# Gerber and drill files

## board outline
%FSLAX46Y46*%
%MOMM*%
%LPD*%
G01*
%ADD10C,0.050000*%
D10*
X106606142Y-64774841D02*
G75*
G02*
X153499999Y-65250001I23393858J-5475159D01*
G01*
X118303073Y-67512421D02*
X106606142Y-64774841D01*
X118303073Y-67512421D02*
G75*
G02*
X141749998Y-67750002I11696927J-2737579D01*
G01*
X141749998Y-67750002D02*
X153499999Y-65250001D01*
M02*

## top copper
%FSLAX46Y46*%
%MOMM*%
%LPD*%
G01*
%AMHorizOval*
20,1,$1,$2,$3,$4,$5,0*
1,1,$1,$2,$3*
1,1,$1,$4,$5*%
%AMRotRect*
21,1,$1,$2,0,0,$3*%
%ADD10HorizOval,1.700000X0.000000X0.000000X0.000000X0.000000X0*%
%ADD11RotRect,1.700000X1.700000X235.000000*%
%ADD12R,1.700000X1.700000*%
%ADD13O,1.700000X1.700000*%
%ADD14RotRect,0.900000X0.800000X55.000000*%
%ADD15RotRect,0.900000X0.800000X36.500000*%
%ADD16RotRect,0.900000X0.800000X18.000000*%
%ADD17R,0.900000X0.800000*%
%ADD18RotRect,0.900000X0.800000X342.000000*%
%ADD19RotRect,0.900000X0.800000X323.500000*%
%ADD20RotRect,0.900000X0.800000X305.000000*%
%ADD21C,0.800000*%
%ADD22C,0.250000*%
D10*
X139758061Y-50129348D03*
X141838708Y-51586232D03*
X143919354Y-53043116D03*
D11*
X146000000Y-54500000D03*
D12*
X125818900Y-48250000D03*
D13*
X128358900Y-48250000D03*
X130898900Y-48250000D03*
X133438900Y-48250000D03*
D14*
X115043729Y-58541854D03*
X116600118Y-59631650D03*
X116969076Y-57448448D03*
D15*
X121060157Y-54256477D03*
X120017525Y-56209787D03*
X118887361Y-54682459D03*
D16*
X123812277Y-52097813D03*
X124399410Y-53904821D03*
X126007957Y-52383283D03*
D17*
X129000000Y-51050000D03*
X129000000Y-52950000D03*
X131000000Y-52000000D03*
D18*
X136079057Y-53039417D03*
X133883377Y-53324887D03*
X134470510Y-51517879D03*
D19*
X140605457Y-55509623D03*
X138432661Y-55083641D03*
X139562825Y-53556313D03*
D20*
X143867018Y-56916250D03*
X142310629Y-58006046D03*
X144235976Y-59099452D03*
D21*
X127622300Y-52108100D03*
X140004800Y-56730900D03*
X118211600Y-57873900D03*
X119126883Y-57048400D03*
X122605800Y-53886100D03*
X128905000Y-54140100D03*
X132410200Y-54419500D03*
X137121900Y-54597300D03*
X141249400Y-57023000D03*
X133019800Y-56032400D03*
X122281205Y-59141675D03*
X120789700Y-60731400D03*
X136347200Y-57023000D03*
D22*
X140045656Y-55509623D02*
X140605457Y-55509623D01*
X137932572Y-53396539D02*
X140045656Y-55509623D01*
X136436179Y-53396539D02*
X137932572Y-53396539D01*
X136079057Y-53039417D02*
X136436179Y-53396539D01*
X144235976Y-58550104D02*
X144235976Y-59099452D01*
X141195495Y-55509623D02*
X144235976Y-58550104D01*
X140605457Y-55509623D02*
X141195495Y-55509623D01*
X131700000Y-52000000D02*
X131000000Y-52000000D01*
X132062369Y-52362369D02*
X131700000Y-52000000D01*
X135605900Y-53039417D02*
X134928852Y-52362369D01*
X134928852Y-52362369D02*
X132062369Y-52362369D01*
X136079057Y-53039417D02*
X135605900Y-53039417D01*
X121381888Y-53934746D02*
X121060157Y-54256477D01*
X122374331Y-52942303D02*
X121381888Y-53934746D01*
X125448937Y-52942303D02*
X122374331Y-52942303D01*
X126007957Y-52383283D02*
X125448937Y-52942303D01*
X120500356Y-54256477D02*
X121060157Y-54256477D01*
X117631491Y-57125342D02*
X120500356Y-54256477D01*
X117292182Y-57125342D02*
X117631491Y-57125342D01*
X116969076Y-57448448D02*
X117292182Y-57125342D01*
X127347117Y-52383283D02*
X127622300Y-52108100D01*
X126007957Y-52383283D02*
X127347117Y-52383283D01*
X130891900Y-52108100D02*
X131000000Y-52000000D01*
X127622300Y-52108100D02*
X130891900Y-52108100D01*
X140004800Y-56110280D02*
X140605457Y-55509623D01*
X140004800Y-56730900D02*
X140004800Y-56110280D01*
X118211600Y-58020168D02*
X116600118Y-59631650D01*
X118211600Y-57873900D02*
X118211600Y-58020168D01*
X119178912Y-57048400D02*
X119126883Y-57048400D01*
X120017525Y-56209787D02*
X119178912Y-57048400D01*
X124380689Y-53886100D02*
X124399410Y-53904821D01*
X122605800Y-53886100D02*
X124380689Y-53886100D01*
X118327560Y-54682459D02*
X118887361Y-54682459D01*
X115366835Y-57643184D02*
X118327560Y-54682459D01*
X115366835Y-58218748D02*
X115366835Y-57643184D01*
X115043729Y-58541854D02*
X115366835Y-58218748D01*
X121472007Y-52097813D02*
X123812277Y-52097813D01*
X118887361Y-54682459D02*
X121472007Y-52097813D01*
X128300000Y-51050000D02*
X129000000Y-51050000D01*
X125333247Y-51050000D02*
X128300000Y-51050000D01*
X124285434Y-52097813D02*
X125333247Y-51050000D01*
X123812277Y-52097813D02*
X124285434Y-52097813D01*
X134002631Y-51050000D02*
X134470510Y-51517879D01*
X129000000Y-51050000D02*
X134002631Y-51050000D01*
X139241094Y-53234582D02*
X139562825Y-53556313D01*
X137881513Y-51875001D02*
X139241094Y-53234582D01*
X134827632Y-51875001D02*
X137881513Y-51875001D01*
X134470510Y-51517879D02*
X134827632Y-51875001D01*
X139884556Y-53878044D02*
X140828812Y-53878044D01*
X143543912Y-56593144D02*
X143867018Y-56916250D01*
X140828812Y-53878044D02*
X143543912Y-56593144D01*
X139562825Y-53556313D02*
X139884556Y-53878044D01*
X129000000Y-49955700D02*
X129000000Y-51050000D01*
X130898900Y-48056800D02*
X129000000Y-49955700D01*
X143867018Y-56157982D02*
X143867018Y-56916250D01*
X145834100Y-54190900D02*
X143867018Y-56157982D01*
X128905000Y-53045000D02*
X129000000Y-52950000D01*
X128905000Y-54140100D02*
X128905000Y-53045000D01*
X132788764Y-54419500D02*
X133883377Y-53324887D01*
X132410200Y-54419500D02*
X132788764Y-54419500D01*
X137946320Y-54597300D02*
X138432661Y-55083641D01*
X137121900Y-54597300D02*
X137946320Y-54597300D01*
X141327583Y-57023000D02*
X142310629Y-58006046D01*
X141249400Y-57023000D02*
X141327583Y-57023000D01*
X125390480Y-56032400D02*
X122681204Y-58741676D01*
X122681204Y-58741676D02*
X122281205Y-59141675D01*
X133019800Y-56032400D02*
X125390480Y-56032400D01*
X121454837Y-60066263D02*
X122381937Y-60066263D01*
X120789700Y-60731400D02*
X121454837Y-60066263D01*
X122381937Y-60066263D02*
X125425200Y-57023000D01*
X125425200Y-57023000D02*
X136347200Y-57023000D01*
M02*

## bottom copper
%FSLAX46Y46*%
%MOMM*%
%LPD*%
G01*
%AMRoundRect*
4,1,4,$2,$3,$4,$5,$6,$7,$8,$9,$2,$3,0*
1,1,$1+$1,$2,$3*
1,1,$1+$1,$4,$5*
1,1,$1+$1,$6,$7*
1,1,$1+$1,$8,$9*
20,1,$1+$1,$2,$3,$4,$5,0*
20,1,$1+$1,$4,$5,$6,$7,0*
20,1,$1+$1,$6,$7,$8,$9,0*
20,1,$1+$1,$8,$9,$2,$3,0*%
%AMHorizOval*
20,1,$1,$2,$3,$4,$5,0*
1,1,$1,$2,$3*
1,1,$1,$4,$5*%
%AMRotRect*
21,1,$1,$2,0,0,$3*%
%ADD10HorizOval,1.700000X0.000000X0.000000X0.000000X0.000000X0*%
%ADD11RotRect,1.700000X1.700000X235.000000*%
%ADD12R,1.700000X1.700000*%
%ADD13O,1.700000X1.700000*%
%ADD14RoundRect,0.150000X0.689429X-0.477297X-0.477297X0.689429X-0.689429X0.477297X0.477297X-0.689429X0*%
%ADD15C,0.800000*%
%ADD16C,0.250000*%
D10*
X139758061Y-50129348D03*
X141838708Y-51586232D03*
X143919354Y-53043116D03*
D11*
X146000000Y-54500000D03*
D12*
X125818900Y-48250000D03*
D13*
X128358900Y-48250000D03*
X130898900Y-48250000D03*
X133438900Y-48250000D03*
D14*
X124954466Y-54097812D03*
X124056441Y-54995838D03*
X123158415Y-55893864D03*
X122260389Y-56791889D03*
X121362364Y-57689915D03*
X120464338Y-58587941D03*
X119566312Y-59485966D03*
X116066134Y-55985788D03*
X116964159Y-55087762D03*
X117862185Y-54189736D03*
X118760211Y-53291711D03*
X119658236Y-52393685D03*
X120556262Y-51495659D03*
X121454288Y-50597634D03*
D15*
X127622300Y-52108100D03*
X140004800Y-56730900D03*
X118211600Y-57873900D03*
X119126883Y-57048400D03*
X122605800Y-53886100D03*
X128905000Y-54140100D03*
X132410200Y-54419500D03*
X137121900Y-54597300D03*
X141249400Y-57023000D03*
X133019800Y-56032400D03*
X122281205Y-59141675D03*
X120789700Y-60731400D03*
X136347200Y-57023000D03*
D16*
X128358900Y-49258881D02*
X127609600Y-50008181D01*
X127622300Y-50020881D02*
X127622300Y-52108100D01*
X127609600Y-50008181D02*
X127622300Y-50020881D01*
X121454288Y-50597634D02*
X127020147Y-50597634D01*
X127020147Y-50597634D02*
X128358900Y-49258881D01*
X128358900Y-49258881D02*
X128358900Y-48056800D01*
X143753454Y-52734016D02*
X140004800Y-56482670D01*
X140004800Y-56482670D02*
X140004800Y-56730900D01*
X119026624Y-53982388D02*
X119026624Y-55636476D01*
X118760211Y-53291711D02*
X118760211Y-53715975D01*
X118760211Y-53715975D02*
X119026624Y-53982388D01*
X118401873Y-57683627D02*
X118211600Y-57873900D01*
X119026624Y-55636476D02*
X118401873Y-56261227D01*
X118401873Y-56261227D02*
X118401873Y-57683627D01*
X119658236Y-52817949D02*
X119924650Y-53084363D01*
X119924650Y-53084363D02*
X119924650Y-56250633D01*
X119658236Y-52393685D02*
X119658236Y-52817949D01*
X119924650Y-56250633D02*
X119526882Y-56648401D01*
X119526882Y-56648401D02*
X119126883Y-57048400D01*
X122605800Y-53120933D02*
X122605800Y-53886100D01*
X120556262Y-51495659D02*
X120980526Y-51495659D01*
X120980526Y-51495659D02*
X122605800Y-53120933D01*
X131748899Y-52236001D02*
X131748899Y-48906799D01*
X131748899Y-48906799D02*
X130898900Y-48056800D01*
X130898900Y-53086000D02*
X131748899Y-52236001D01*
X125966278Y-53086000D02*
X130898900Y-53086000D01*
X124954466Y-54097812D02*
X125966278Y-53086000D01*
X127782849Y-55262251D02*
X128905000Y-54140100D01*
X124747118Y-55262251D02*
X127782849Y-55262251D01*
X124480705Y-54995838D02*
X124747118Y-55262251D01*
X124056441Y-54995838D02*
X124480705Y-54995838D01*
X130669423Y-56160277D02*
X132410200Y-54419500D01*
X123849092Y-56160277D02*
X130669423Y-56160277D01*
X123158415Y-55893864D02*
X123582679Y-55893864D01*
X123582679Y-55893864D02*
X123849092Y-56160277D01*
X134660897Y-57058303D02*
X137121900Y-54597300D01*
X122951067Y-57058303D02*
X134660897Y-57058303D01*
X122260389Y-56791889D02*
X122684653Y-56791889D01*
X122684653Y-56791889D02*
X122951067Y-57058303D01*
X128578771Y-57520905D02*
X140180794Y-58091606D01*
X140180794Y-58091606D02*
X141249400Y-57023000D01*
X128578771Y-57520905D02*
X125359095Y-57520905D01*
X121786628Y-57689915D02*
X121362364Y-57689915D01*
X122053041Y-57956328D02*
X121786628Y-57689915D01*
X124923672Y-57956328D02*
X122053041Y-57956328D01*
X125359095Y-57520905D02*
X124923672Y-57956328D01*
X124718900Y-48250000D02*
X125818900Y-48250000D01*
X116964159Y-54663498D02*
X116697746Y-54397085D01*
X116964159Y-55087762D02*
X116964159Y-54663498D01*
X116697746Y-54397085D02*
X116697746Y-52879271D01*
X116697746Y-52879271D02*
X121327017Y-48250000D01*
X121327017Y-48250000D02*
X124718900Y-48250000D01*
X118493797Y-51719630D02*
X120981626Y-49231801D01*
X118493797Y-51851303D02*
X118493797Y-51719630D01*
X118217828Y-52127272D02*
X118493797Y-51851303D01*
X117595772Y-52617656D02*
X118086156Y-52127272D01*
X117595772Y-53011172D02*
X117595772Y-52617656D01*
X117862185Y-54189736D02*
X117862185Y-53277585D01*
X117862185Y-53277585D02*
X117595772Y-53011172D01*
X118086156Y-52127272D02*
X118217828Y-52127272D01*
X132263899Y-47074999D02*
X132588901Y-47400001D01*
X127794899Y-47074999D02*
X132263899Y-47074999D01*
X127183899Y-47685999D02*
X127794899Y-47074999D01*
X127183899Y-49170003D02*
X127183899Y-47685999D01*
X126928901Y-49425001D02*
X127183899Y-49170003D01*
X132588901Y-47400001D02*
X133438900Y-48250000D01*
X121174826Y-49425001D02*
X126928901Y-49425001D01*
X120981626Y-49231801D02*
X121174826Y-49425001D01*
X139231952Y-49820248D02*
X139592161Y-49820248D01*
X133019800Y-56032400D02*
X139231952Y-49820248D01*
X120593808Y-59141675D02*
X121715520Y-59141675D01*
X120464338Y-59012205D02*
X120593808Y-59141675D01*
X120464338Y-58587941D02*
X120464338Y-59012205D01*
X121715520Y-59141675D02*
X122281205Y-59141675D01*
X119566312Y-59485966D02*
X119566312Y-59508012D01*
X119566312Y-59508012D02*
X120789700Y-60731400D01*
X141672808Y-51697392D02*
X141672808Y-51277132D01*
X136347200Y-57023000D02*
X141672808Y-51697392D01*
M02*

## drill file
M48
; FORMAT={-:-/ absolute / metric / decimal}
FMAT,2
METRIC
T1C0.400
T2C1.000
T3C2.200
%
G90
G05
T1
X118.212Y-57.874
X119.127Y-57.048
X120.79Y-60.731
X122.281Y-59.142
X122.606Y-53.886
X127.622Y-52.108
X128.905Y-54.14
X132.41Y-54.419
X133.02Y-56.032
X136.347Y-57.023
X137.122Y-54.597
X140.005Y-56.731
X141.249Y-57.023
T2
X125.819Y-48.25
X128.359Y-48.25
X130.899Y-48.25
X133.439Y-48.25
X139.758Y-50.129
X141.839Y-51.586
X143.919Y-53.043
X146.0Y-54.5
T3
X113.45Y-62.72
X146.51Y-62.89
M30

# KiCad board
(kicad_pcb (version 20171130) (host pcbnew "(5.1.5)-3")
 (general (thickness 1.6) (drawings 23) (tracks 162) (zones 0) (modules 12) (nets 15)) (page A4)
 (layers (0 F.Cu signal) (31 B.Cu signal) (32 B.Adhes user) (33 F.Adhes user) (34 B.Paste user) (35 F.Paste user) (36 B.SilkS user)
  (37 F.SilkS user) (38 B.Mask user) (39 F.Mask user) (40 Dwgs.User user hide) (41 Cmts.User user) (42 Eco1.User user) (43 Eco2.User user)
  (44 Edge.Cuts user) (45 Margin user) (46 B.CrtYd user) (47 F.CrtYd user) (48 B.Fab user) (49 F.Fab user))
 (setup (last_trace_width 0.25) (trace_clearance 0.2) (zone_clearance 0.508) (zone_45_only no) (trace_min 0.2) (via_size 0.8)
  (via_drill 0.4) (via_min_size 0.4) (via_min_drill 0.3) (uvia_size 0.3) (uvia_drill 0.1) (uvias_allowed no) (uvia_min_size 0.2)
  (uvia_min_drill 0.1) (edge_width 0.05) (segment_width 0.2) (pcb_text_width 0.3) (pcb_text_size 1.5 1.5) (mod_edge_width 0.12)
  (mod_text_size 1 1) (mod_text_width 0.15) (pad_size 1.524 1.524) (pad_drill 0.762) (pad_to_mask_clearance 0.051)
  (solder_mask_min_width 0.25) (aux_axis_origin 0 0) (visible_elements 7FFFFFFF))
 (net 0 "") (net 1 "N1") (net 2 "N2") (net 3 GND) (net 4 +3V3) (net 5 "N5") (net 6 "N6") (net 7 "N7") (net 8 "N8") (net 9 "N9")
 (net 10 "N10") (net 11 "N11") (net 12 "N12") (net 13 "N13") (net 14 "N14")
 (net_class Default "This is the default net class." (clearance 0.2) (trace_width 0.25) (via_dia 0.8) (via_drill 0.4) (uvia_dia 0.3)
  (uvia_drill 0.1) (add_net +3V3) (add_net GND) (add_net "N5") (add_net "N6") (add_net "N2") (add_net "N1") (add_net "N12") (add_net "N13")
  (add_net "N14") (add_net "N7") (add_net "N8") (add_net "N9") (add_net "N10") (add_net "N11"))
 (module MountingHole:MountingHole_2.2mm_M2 (layer F.Cu) (at 146.51 62.89)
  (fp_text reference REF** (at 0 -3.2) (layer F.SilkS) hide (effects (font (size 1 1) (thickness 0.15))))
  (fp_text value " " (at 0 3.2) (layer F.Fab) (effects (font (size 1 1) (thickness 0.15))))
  (pad 1 np_thru_hole circle (at 0 0) (size 2.2 2.2) (drill 2.2) (layers *.Cu *.Mask)))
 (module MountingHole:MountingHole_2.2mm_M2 (layer F.Cu) (at 113.45 62.72)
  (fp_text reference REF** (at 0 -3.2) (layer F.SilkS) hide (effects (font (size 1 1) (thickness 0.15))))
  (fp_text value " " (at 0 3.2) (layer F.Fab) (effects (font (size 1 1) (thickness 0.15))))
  (pad 1 np_thru_hole circle (at 0 0) (size 2.2 2.2) (drill 2.2) (layers *.Cu *.Mask)))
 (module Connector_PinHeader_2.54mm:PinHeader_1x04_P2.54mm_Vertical (layer F.Cu) (at 146 54.5 235)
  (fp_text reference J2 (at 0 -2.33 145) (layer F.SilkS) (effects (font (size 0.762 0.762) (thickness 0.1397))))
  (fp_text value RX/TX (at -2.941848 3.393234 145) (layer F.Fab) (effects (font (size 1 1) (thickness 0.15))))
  (pad 4 thru_hole oval (at 0 7.62 235) (size 1.7 1.7) (drill 1) (layers *.Cu *.Mask) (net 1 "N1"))
  (pad 3 thru_hole oval (at 0 5.08 235) (size 1.7 1.7) (drill 1) (layers *.Cu *.Mask) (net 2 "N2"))
  (pad 2 thru_hole oval (at 0 2.54 235) (size 1.7 1.7) (drill 1) (layers *.Cu *.Mask) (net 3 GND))
  (pad 1 thru_hole rect (at 0 0 235) (size 1.7 1.7) (drill 1) (layers *.Cu *.Mask) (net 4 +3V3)))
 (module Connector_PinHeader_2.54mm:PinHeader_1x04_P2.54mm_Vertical (layer F.Cu) (at 125.8189 48.25 90)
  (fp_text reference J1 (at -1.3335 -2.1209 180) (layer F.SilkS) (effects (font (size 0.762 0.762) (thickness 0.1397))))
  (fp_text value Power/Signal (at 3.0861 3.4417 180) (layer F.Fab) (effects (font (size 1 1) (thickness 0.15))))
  (pad 1 thru_hole rect (at 0 0 90) (size 1.7 1.7) (drill 1) (layers *.Cu *.Mask) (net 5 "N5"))
  (pad 2 thru_hole oval (at 0 2.54 90) (size 1.7 1.7) (drill 1) (layers *.Cu *.Mask) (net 3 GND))
  (pad 3 thru_hole oval (at 0 5.08 90) (size 1.7 1.7) (drill 1) (layers *.Cu *.Mask) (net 4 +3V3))
  (pad 4 thru_hole oval (at 0 7.62 90) (size 1.7 1.7) (drill 1) (layers *.Cu *.Mask) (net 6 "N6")))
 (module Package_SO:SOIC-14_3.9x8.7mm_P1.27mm (layer B.Cu) (at 120.5103 55.0418 135)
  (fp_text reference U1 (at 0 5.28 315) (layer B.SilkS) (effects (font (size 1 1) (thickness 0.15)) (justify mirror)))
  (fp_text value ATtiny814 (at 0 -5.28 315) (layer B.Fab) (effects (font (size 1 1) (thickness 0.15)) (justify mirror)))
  (pad 1 smd roundrect (at -2.475 3.81 135) (size 1.95 0.6) (layers B.Cu B.Paste B.Mask) (roundrect_rratio 0.25) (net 4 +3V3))
  (pad 2 smd roundrect (at -2.475 2.54 135) (size 1.95 0.6) (layers B.Cu B.Paste B.Mask) (roundrect_rratio 0.25) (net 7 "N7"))
  (pad 3 smd roundrect (at -2.475 1.27 135) (size 1.95 0.6) (layers B.Cu B.Paste B.Mask) (roundrect_rratio 0.25) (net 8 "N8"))
  (pad 4 smd roundrect (at -2.475 0 135) (size 1.95 0.6) (layers B.Cu B.Paste B.Mask) (roundrect_rratio 0.25) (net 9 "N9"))
  (pad 5 smd roundrect (at -2.475 -1.27 135) (size 1.95 0.6) (layers B.Cu B.Paste B.Mask) (roundrect_rratio 0.25) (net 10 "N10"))
  (pad 6 smd roundrect (at -2.475 -2.54 135) (size 1.95 0.6) (layers B.Cu B.Paste B.Mask) (roundrect_rratio 0.25) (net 1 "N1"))
  (pad 7 smd roundrect (at -2.475 -3.81 135) (size 1.95 0.6) (layers B.Cu B.Paste B.Mask) (roundrect_rratio 0.25) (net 2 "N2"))
  (pad 8 smd roundrect (at 2.475 -3.81 135) (size 1.95 0.6) (layers B.Cu B.Paste B.Mask) (roundrect_rratio 0.25) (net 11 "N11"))
  (pad 9 smd roundrect (at 2.475 -2.54 135) (size 1.95 0.6) (layers B.Cu B.Paste B.Mask) (roundrect_rratio 0.25) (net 5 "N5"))
  (pad 10 smd roundrect (at 2.475 -1.27 135) (size 1.95 0.6) (layers B.Cu B.Paste B.Mask) (roundrect_rratio 0.25) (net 6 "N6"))
  (pad 11 smd roundrect (at 2.475 0 135) (size 1.95 0.6) (layers B.Cu B.Paste B.Mask) (roundrect_rratio 0.25) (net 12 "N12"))
  (pad 12 smd roundrect (at 2.475 1.27 135) (size 1.95 0.6) (layers B.Cu B.Paste B.Mask) (roundrect_rratio 0.25) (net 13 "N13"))
  (pad 13 smd roundrect (at 2.475 2.54 135) (size 1.95 0.6) (layers B.Cu B.Paste B.Mask) (roundrect_rratio 0.25) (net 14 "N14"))
  (pad 14 smd roundrect (at 2.475 3.81 135) (size 1.95 0.6) (layers B.Cu B.Paste B.Mask) (roundrect_rratio 0.25) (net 3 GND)))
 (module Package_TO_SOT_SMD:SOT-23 (layer F.Cu) (at 116.3955 58.2676 55)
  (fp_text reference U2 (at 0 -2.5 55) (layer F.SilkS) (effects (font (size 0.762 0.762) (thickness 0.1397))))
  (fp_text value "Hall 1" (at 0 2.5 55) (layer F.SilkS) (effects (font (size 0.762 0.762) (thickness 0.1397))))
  (pad 1 smd rect (at -1 -0.95 55) (size 0.9 0.8) (layers F.Cu F.Paste F.Mask) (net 4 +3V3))
  (pad 2 smd rect (at -1 0.95 55) (size 0.9 0.8) (layers F.Cu F.Paste F.Mask) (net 12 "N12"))
  (pad 3 smd rect (at 1 0 55) (size 0.9 0.8) (layers F.Cu F.Paste F.Mask) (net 3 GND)))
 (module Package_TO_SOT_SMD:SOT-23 (layer F.Cu) (at 120.2563 54.8513 36.5)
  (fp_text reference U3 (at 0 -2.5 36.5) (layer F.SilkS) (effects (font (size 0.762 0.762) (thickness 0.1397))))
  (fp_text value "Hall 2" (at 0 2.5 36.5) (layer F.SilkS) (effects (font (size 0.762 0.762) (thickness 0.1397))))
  (pad 3 smd rect (at 1 0 36.5) (size 0.9 0.8) (layers F.Cu F.Paste F.Mask) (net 3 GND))
  (pad 2 smd rect (at -1 0.95 36.5) (size 0.9 0.8) (layers F.Cu F.Paste F.Mask) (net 13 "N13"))
  (pad 1 smd rect (at -1 -0.95 36.5) (size 0.9 0.8) (layers F.Cu F.Paste F.Mask) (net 4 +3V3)))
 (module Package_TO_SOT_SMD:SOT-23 (layer F.Cu) (at 125.0569 52.6923 18)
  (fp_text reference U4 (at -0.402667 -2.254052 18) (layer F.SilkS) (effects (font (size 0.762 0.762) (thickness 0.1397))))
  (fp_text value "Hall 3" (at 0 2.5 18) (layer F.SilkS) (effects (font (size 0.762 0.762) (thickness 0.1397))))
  (pad 1 smd rect (at -1 -0.95 18) (size 0.9 0.8) (layers F.Cu F.Paste F.Mask) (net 4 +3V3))
  (pad 2 smd rect (at -1 0.95 18) (size 0.9 0.8) (layers F.Cu F.Paste F.Mask) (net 14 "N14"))
  (pad 3 smd rect (at 1 0 18) (size 0.9 0.8) (layers F.Cu F.Paste F.Mask) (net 3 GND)))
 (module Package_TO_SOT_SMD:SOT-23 (layer F.Cu) (at 130 52)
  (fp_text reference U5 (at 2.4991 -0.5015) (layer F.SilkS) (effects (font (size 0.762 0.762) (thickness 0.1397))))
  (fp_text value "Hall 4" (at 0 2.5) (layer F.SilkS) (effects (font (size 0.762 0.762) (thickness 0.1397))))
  (pad 1 smd rect (at -1 -0.95) (size 0.9 0.8) (layers F.Cu F.Paste F.Mask) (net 4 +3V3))
  (pad 2 smd rect (at -1 0.95) (size 0.9 0.8) (layers F.Cu F.Paste F.Mask) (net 7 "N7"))
  (pad 3 smd rect (at 1 0) (size 0.9 0.8) (layers F.Cu F.Paste F.Mask) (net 3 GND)))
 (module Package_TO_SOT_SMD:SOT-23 (layer F.Cu) (at 135.128 52.7304 342)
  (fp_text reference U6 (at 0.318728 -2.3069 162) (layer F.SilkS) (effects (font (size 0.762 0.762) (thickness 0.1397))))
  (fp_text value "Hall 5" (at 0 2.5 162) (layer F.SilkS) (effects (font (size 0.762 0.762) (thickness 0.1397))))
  (pad 3 smd rect (at 1 0 342) (size 0.9 0.8) (layers F.Cu F.Paste F.Mask) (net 3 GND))
  (pad 2 smd rect (at -1 0.95 342) (size 0.9 0.8) (layers F.Cu F.Paste F.Mask) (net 8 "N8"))
  (pad 1 smd rect (at -1 -0.95 342) (size 0.9 0.8) (layers F.Cu F.Paste F.Mask) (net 4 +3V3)))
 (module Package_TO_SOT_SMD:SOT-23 (layer F.Cu) (at 139.8016 54.9148 323.5)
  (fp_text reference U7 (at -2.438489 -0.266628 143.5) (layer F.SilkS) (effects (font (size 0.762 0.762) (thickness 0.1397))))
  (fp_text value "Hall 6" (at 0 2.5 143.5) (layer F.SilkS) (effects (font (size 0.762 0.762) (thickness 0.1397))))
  (pad 3 smd rect (at 1 0 323.5) (size 0.9 0.8) (layers F.Cu F.Paste F.Mask) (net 3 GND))
  (pad 2 smd rect (at -1 0.95 323.5) (size 0.9 0.8) (layers F.Cu F.Paste F.Mask) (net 9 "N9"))
  (pad 1 smd rect (at -1 -0.95 323.5) (size 0.9 0.8) (layers F.Cu F.Paste F.Mask) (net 4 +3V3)))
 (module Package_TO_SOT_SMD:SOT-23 (layer F.Cu) (at 143.6624 58.2803 305)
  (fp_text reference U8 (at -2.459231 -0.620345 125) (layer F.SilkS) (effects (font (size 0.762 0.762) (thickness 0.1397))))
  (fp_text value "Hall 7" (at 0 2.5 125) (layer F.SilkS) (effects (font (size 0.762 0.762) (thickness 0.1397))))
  (pad 1 smd rect (at -1 -0.95 305) (size 0.9 0.8) (layers F.Cu F.Paste F.Mask) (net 4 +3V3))
  (pad 2 smd rect (at -1 0.95 305) (size 0.9 0.8) (layers F.Cu F.Paste F.Mask) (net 10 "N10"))
  (pad 3 smd rect (at 1 0 305) (size 0.9 0.8) (layers F.Cu F.Paste F.Mask) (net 3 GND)))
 (gr_arc (start 130 70.25) (end 153.499999 65.250001) (angle -154.8159682) (layer Edge.Cuts) (width 0.05))
 (gr_line (start 118.303073 67.512421) (end 106.606142 64.774841) (layer Edge.Cuts) (width 0.05))
 (gr_arc (start 130 70.25) (end 141.749998 67.750002) (angle -154.8159719) (layer Edge.Cuts) (width 0.05))
 (gr_line (start 141.749998 67.750002) (end 153.499999 65.250001) (layer Edge.Cuts) (width 0.05))
 (segment (start 140.045656 55.509623) (end 140.605457 55.509623) (width 0.25) (layer F.Cu) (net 3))
 (segment (start 137.932572 53.396539) (end 140.045656 55.509623) (width 0.25) (layer F.Cu) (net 3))
 (segment (start 136.436179 53.396539) (end 137.932572 53.396539) (width 0.25) (layer F.Cu) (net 3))
 (segment (start 136.079057 53.039417) (end 136.436179 53.396539) (width 0.25) (layer F.Cu) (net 3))
 (segment (start 144.235976 58.550104) (end 144.235976 59.099452) (width 0.25) (layer F.Cu) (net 3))
 (segment (start 141.195495 55.509623) (end 144.235976 58.550104) (width 0.25) (layer F.Cu) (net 3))
 (segment (start 140.605457 55.509623) (end 141.195495 55.509623) (width 0.25) (layer F.Cu) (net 3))
 (segment (start 131.7 52) (end 131 52) (width 0.25) (layer F.Cu) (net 3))
 (segment (start 132.062369 52.362369) (end 131.7 52) (width 0.25) (layer F.Cu) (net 3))
 (segment (start 135.6059 53.039417) (end 134.928852 52.362369) (width 0.25) (layer F.Cu) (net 3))
 (segment (start 134.928852 52.362369) (end 132.062369 52.362369) (width 0.25) (layer F.Cu) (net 3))
 (segment (start 136.079057 53.039417) (end 135.6059 53.039417) (width 0.25) (layer F.Cu) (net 3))
 (segment (start 121.381888 53.934746) (end 121.060157 54.256477) (width 0.25) (layer F.Cu) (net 3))
 (segment (start 122.374331 52.942303) (end 121.381888 53.934746) (width 0.25) (layer F.Cu) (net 3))
 (segment (start 125.448937 52.942303) (end 122.374331 52.942303) (width 0.25) (layer F.Cu) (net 3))
 (segment (start 126.007957 52.383283) (end 125.448937 52.942303) (width 0.25) (layer F.Cu) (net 3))
 (segment (start 120.500356 54.256477) (end 121.060157 54.256477) (width 0.25) (layer F.Cu) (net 3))
 (segment (start 117.631491 57.125342) (end 120.500356 54.256477) (width 0.25) (layer F.Cu) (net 3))
 (segment (start 117.292182 57.125342) (end 117.631491 57.125342) (width 0.25) (layer F.Cu) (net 3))
 (segment (start 116.969076 57.448448) (end 117.292182 57.125342) (width 0.25) (layer F.Cu) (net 3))
 (segment (start 128.3589 49.258881) (end 127.6096 50.008181) (width 0.25) (layer B.Cu) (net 3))
 (via (at 127.6223 52.1081) (size 0.8) (drill 0.4) (layers F.Cu B.Cu) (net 3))
 (segment (start 127.6223 50.020881) (end 127.6223 52.1081) (width 0.25) (layer B.Cu) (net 3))
 (segment (start 127.6096 50.008181) (end 127.6223 50.020881) (width 0.25) (layer B.Cu) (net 3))
 (segment (start 127.347117 52.383283) (end 127.6223 52.1081) (width 0.25) (layer F.Cu) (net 3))
 (segment (start 126.007957 52.383283) (end 127.347117 52.383283) (width 0.25) (layer F.Cu) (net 3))
 (segment (start 130.8919 52.1081) (end 131 52) (width 0.25) (layer F.Cu) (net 3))
 (segment (start 127.6223 52.1081) (end 130.8919 52.1081) (width 0.25) (layer F.Cu) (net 3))
 (segment (start 121.454288 50.597634) (end 127.020147 50.597634) (width 0.25) (layer B.Cu) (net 3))
 (segment (start 127.020147 50.597634) (end 128.3589 49.258881) (width 0.25) (layer B.Cu) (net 3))
 (segment (start 128.3589 49.258881) (end 128.3589 48.0568) (width 0.25) (layer B.Cu) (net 3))
 (via (at 140.0048 56.7309) (size 0.8) (drill 0.4) (layers F.Cu B.Cu) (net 3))
 (segment (start 143.753454 52.734016) (end 140.0048 56.48267) (width 0.25) (layer B.Cu) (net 3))
 (segment (start 140.0048 56.48267) (end 140.0048 56.7309) (width 0.25) (layer B.Cu) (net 3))
 (segment (start 140.0048 56.11028) (end 140.605457 55.509623) (width 0.25) (layer F.Cu) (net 3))
 (segment (start 140.0048 56.7309) (end 140.0048 56.11028) (width 0.25) (layer F.Cu) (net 3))
 (segment (start 119.026624 53.982388) (end 119.026624 55.636476) (width 0.25) (layer B.Cu) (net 12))
 (segment (start 118.760211 53.291711) (end 118.760211 53.715975) (width 0.25) (layer B.Cu) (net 12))
 (segment (start 118.760211 53.715975) (end 119.026624 53.982388) (width 0.25) (layer B.Cu) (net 12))
 (via (at 118.2116 57.8739) (size 0.8) (drill 0.4) (layers F.Cu B.Cu) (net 12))
 (segment (start 118.401873 57.683627) (end 118.2116 57.8739) (width 0.25) (layer B.Cu) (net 12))
 (segment (start 119.026624 55.636476) (end 118.401873 56.261227) (width 0.25) (layer B.Cu) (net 12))
 (segment (start 118.401873 56.261227) (end 118.401873 57.683627) (width 0.25) (layer B.Cu) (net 12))
 (segment (start 118.2116 58.020168) (end 116.600118 59.63165) (width 0.25) (layer F.Cu) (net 12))
 (segment (start 118.2116 57.8739) (end 118.2116 58.020168) (width 0.25) (layer F.Cu) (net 12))
 (segment (start 119.658236 52.817949) (end 119.92465 53.084363) (width 0.25) (layer B.Cu) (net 13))
 (segment (start 119.92465 53.084363) (end 119.92465 56.250633) (width 0.25) (layer B.Cu) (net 13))
 (segment (start 119.658236 52.393685) (end 119.658236 52.817949) (width 0.25) (layer B.Cu) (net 13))
 (segment (start 119.92465 56.250633) (end 119.526882 56.648401) (width 0.25) (layer B.Cu) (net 13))
 (segment (start 119.178912 57.0484) (end 119.126883 57.0484) (width 0.25) (layer F.Cu) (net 13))
 (segment (start 119.526882 56.648401) (end 119.126883 57.0484) (width 0.25) (layer B.Cu) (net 13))
 (via (at 119.126883 57.0484) (size 0.8) (drill 0.4) (layers F.Cu B.Cu) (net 13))
 (segment (start 120.017525 56.209787) (end 119.178912 57.0484) (width 0.25) (layer F.Cu) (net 13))
 (via (at 122.6058 53.8861) (size 0.8) (drill 0.4) (layers F.Cu B.Cu) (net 14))
 (segment (start 122.6058 53.120933) (end 122.6058 53.8861) (width 0.25) (layer B.Cu) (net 14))
 (segment (start 120.556262 51.495659) (end 120.980526 51.495659) (width 0.25) (layer B.Cu) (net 14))
 (segment (start 120.980526 51.495659) (end 122.6058 53.120933) (width 0.25) (layer B.Cu) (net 14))
 (segment (start 124.380689 53.8861) (end 124.39941 53.904821) (width 0.25) (layer F.Cu) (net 14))
 (segment (start 122.6058 53.8861) (end 124.380689 53.8861) (width 0.25) (layer F.Cu) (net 14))
 (segment (start 118.32756 54.682459) (end 118.887361 54.682459) (width 0.25) (layer F.Cu) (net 4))
 (segment (start 115.366835 57.643184) (end 118.32756 54.682459) (width 0.25) (layer F.Cu) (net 4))
 (segment (start 115.366835 58.218748) (end 115.366835 57.643184) (width 0.25) (layer F.Cu) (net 4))
 (segment (start 115.043729 58.541854) (end 115.366835 58.218748) (width 0.25) (layer F.Cu) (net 4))
 (segment (start 121.472007 52.097813) (end 123.812277 52.097813) (width 0.25) (layer F.Cu) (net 4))
 (segment (start 118.887361 54.682459) (end 121.472007 52.097813) (width 0.25) (layer F.Cu) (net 4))
 (segment (start 128.3 51.05) (end 129 51.05) (width 0.25) (layer F.Cu) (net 4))
 (segment (start 125.333247 51.05) (end 128.3 51.05) (width 0.25) (layer F.Cu) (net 4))
 (segment (start 124.285434 52.097813) (end 125.333247 51.05) (width 0.25) (layer F.Cu) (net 4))
 (segment (start 123.812277 52.097813) (end 124.285434 52.097813) (width 0.25) (layer F.Cu) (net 4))
 (segment (start 134.002631 51.05) (end 134.47051 51.517879) (width 0.25) (layer F.Cu) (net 4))
 (segment (start 129 51.05) (end 134.002631 51.05) (width 0.25) (layer F.Cu) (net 4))
 (segment (start 139.241094 53.234582) (end 139.562825 53.556313) (width 0.25) (layer F.Cu) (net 4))
 (segment (start 137.881513 51.875001) (end 139.241094 53.234582) (width 0.25) (layer F.Cu) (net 4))
 (segment (start 134.827632 51.875001) (end 137.881513 51.875001) (width 0.25) (layer F.Cu) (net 4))
 (segment (start 134.47051 51.517879) (end 134.827632 51.875001) (width 0.25) (layer F.Cu) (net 4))
 (segment (start 139.884556 53.878044) (end 140.828812 53.878044) (width 0.25) (layer F.Cu) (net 4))
 (segment (start 143.543912 56.593144) (end 143.867018 56.91625) (width 0.25) (layer F.Cu) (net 4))
 (segment (start 140.828812 53.878044) (end 143.543912 56.593144) (width 0.25) (layer F.Cu) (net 4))
 (segment (start 139.562825 53.556313) (end 139.884556 53.878044) (width 0.25) (layer F.Cu) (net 4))
 (segment (start 129 49.9557) (end 129 51.05) (width 0.25) (layer F.Cu) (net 4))
 (segment (start 130.8989 48.0568) (end 129 49.9557) (width 0.25) (layer F.Cu) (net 4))
 (segment (start 131.748899 52.236001) (end 131.748899 48.906799) (width 0.25) (layer B.Cu) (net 4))
 (segment (start 131.748899 48.906799) (end 130.8989 48.0568) (width 0.25) (layer B.Cu) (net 4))
 (segment (start 130.8989 53.086) (end 131.748899 52.236001) (width 0.25) (layer B.Cu) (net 4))
 (segment (start 125.966278 53.086) (end 130.8989 53.086) (width 0.25) (layer B.Cu) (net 4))
 (segment (start 124.954466 54.097812) (end 125.966278 53.086) (width 0.25) (layer B.Cu) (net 4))
 (segment (start 143.867018 56.157982) (end 143.867018 56.91625) (width 0.25) (layer F.Cu) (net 4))
 (segment (start 145.8341 54.1909) (end 143.867018 56.157982) (width 0.25) (layer F.Cu) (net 4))
 (segment (start 127.782849 55.262251) (end 128.905 54.1401) (width 0.25) (layer B.Cu) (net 7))
 (segment (start 124.747118 55.262251) (end 127.782849 55.262251) (width 0.25) (layer B.Cu) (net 7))
 (segment (start 124.480705 54.995838) (end 124.747118 55.262251) (width 0.25) (layer B.Cu) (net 7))
 (via (at 128.905 54.1401) (size 0.8) (drill 0.4) (layers F.Cu B.Cu) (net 7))
 (segment (start 124.056441 54.995838) (end 124.480705 54.995838) (width 0.25) (layer B.Cu) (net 7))
 (segment (start 128.905 53.045) (end 129 52.95) (width 0.25) (layer F.Cu) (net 7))
 (segment (start 128.905 54.1401) (end 128.905 53.045) (width 0.25) (layer F.Cu) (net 7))
 (via (at 132.4102 54.4195) (size 0.8) (drill 0.4) (layers F.Cu B.Cu) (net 8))
 (segment (start 130.669423 56.160277) (end 132.4102 54.4195) (width 0.25) (layer B.Cu) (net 8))
 (segment (start 123.849092 56.160277) (end 130.669423 56.160277) (width 0.25) (layer B.Cu) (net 8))
 (segment (start 123.158415 55.893864) (end 123.582679 55.893864) (width 0.25) (layer B.Cu) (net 8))
 (segment (start 123.582679 55.893864) (end 123.849092 56.160277) (width 0.25) (layer B.Cu) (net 8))
 (segment (start 132.788764 54.4195) (end 133.883377 53.324887) (width 0.25) (layer F.Cu) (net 8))
 (segment (start 132.4102 54.4195) (end 132.788764 54.4195) (width 0.25) (layer F.Cu) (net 8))
 (via (at 137.1219 54.5973) (size 0.8) (drill 0.4) (layers F.Cu B.Cu) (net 9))
 (segment (start 134.660897 57.058303) (end 137.1219 54.5973) (width 0.25) (layer B.Cu) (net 9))
 (segment (start 122.951067 57.058303) (end 134.660897 57.058303) (width 0.25) (layer B.Cu) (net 9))
 (segment (start 122.260389 56.791889) (end 122.684653 56.791889) (width 0.25) (layer B.Cu) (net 9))
 (segment (start 122.684653 56.791889) (end 122.951067 57.058303) (width 0.25) (layer B.Cu) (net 9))
 (segment (start 137.94632 54.5973) (end 138.432661 55.083641) (width 0.25) (layer F.Cu) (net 9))
 (segment (start 137.1219 54.5973) (end 137.94632 54.5973) (width 0.25) (layer F.Cu) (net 9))
 (via (at 141.2494 57.023) (size 0.8) (drill 0.4) (layers F.Cu B.Cu) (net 10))
 (segment (start 128.578771 57.520905) (end 140.180794 58.091606) (width 0.25) (layer B.Cu) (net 10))
 (segment (start 140.180794 58.091606) (end 141.2494 57.023) (width 0.25) (layer B.Cu) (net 10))
 (segment (start 141.327583 57.023) (end 142.310629 58.006046) (width 0.25) (layer F.Cu) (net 10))
 (segment (start 141.2494 57.023) (end 141.327583 57.023) (width 0.25) (layer F.Cu) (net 10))
 (segment (start 128.578771 57.520905) (end 125.359095 57.520905) (width 0.25) (layer B.Cu) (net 10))
 (segment (start 121.786628 57.689915) (end 121.362364 57.689915) (width 0.25) (layer B.Cu) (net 10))
 (segment (start 122.053041 57.956328) (end 121.786628 57.689915) (width 0.25) (layer B.Cu) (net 10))
 (segment (start 124.923672 57.956328) (end 122.053041 57.956328) (width 0.25) (layer B.Cu) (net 10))
 (segment (start 125.359095 57.520905) (end 124.923672 57.956328) (width 0.25) (layer B.Cu) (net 10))
 (segment (start 124.7189 48.25) (end 125.8189 48.25) (width 0.25) (layer B.Cu) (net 5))
 (segment (start 116.964159 54.663498) (end 116.697746 54.397085) (width 0.25) (layer B.Cu) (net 5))
 (segment (start 116.964159 55.087762) (end 116.964159 54.663498) (width 0.25) (layer B.Cu) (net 5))
 (segment (start 116.697746 54.397085) (end 116.697746 52.879271) (width 0.25) (layer B.Cu) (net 5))
 (segment (start 116.697746 52.879271) (end 121.327017 48.25) (width 0.25) (layer B.Cu) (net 5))
 (segment (start 121.327017 48.25) (end 124.7189 48.25) (width 0.25) (layer B.Cu) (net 5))
 (segment (start 118.493797 51.71963) (end 120.981626 49.231801) (width 0.25) (layer B.Cu) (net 6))
 (segment (start 118.493797 51.851303) (end 118.493797 51.71963) (width 0.25) (layer B.Cu) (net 6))
 (segment (start 118.217828 52.127272) (end 118.493797 51.851303) (width 0.25) (layer B.Cu) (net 6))
 (segment (start 117.595772 52.617656) (end 118.086156 52.127272) (width 0.25) (layer B.Cu) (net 6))
 (segment (start 117.595772 53.011172) (end 117.595772 52.617656) (width 0.25) (layer B.Cu) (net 6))
 (segment (start 117.862185 54.189736) (end 117.862185 53.277585) (width 0.25) (layer B.Cu) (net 6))
 (segment (start 117.862185 53.277585) (end 117.595772 53.011172) (width 0.25) (layer B.Cu) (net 6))
 (segment (start 118.086156 52.127272) (end 118.217828 52.127272) (width 0.25) (layer B.Cu) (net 6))
 (segment (start 132.263899 47.074999) (end 132.588901 47.400001) (width 0.25) (layer B.Cu) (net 6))
 (segment (start 127.794899 47.074999) (end 132.263899 47.074999) (width 0.25) (layer B.Cu) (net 6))
 (segment (start 127.183899 47.685999) (end 127.794899 47.074999) (width 0.25) (layer B.Cu) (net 6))
 (segment (start 127.183899 49.170003) (end 127.183899 47.685999) (width 0.25) (layer B.Cu) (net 6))
 (segment (start 126.928901 49.425001) (end 127.183899 49.170003) (width 0.25) (layer B.Cu) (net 6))
 (segment (start 132.588901 47.400001) (end 133.4389 48.25) (width 0.25) (layer B.Cu) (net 6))
 (segment (start 121.174826 49.425001) (end 126.928901 49.425001) (width 0.25) (layer B.Cu) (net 6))
 (segment (start 120.981626 49.231801) (end 121.174826 49.425001) (width 0.25) (layer B.Cu) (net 6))
 (via (at 133.0198 56.0324) (size 0.8) (drill 0.4) (layers F.Cu B.Cu) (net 1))
 (segment (start 139.231952 49.820248) (end 139.592161 49.820248) (width 0.25) (layer B.Cu) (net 1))
 (segment (start 133.0198 56.0324) (end 139.231952 49.820248) (width 0.25) (layer B.Cu) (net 1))
 (segment (start 120.593808 59.141675) (end 121.71552 59.141675) (width 0.25) (layer B.Cu) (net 1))
 (segment (start 125.39048 56.0324) (end 122.681204 58.741676) (width 0.25) (layer F.Cu) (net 1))
 (segment (start 122.681204 58.741676) (end 122.281205 59.141675) (width 0.25) (layer F.Cu) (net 1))
 (segment (start 133.0198 56.0324) (end 125.39048 56.0324) (width 0.25) (layer F.Cu) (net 1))
 (segment (start 120.464338 59.012205) (end 120.593808 59.141675) (width 0.25) (layer B.Cu) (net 1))
 (via (at 122.281205 59.141675) (size 0.8) (drill 0.4) (layers F.Cu B.Cu) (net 1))
 (segment (start 120.464338 58.587941) (end 120.464338 59.012205) (width 0.25) (layer B.Cu) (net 1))
 (segment (start 121.71552 59.141675) (end 122.281205 59.141675) (width 0.25) (layer B.Cu) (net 1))
 (via (at 120.7897 60.7314) (size 0.8) (drill 0.4) (layers F.Cu B.Cu) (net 2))
 (segment (start 119.566312 59.485966) (end 119.566312 59.508012) (width 0.25) (layer B.Cu) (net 2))
 (segment (start 119.566312 59.508012) (end 120.7897 60.7314) (width 0.25) (layer B.Cu) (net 2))
 (segment (start 121.454837 60.066263) (end 122.381937 60.066263) (width 0.25) (layer F.Cu) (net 2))
 (segment (start 120.7897 60.7314) (end 121.454837 60.066263) (width 0.25) (layer F.Cu) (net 2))
 (via (at 136.3472 57.023) (size 0.8) (drill 0.4) (layers F.Cu B.Cu) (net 2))
 (segment (start 122.381937 60.066263) (end 125.4252 57.023) (width 0.25) (layer F.Cu) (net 2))
 (segment (start 125.4252 57.023) (end 136.3472 57.023) (width 0.25) (layer F.Cu) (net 2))
 (segment (start 141.672808 51.697392) (end 141.672808 51.277132) (width 0.25) (layer B.Cu) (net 2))
 (segment (start 136.3472 57.023) (end 141.672808 51.697392) (width 0.25) (layer B.Cu) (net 2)))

